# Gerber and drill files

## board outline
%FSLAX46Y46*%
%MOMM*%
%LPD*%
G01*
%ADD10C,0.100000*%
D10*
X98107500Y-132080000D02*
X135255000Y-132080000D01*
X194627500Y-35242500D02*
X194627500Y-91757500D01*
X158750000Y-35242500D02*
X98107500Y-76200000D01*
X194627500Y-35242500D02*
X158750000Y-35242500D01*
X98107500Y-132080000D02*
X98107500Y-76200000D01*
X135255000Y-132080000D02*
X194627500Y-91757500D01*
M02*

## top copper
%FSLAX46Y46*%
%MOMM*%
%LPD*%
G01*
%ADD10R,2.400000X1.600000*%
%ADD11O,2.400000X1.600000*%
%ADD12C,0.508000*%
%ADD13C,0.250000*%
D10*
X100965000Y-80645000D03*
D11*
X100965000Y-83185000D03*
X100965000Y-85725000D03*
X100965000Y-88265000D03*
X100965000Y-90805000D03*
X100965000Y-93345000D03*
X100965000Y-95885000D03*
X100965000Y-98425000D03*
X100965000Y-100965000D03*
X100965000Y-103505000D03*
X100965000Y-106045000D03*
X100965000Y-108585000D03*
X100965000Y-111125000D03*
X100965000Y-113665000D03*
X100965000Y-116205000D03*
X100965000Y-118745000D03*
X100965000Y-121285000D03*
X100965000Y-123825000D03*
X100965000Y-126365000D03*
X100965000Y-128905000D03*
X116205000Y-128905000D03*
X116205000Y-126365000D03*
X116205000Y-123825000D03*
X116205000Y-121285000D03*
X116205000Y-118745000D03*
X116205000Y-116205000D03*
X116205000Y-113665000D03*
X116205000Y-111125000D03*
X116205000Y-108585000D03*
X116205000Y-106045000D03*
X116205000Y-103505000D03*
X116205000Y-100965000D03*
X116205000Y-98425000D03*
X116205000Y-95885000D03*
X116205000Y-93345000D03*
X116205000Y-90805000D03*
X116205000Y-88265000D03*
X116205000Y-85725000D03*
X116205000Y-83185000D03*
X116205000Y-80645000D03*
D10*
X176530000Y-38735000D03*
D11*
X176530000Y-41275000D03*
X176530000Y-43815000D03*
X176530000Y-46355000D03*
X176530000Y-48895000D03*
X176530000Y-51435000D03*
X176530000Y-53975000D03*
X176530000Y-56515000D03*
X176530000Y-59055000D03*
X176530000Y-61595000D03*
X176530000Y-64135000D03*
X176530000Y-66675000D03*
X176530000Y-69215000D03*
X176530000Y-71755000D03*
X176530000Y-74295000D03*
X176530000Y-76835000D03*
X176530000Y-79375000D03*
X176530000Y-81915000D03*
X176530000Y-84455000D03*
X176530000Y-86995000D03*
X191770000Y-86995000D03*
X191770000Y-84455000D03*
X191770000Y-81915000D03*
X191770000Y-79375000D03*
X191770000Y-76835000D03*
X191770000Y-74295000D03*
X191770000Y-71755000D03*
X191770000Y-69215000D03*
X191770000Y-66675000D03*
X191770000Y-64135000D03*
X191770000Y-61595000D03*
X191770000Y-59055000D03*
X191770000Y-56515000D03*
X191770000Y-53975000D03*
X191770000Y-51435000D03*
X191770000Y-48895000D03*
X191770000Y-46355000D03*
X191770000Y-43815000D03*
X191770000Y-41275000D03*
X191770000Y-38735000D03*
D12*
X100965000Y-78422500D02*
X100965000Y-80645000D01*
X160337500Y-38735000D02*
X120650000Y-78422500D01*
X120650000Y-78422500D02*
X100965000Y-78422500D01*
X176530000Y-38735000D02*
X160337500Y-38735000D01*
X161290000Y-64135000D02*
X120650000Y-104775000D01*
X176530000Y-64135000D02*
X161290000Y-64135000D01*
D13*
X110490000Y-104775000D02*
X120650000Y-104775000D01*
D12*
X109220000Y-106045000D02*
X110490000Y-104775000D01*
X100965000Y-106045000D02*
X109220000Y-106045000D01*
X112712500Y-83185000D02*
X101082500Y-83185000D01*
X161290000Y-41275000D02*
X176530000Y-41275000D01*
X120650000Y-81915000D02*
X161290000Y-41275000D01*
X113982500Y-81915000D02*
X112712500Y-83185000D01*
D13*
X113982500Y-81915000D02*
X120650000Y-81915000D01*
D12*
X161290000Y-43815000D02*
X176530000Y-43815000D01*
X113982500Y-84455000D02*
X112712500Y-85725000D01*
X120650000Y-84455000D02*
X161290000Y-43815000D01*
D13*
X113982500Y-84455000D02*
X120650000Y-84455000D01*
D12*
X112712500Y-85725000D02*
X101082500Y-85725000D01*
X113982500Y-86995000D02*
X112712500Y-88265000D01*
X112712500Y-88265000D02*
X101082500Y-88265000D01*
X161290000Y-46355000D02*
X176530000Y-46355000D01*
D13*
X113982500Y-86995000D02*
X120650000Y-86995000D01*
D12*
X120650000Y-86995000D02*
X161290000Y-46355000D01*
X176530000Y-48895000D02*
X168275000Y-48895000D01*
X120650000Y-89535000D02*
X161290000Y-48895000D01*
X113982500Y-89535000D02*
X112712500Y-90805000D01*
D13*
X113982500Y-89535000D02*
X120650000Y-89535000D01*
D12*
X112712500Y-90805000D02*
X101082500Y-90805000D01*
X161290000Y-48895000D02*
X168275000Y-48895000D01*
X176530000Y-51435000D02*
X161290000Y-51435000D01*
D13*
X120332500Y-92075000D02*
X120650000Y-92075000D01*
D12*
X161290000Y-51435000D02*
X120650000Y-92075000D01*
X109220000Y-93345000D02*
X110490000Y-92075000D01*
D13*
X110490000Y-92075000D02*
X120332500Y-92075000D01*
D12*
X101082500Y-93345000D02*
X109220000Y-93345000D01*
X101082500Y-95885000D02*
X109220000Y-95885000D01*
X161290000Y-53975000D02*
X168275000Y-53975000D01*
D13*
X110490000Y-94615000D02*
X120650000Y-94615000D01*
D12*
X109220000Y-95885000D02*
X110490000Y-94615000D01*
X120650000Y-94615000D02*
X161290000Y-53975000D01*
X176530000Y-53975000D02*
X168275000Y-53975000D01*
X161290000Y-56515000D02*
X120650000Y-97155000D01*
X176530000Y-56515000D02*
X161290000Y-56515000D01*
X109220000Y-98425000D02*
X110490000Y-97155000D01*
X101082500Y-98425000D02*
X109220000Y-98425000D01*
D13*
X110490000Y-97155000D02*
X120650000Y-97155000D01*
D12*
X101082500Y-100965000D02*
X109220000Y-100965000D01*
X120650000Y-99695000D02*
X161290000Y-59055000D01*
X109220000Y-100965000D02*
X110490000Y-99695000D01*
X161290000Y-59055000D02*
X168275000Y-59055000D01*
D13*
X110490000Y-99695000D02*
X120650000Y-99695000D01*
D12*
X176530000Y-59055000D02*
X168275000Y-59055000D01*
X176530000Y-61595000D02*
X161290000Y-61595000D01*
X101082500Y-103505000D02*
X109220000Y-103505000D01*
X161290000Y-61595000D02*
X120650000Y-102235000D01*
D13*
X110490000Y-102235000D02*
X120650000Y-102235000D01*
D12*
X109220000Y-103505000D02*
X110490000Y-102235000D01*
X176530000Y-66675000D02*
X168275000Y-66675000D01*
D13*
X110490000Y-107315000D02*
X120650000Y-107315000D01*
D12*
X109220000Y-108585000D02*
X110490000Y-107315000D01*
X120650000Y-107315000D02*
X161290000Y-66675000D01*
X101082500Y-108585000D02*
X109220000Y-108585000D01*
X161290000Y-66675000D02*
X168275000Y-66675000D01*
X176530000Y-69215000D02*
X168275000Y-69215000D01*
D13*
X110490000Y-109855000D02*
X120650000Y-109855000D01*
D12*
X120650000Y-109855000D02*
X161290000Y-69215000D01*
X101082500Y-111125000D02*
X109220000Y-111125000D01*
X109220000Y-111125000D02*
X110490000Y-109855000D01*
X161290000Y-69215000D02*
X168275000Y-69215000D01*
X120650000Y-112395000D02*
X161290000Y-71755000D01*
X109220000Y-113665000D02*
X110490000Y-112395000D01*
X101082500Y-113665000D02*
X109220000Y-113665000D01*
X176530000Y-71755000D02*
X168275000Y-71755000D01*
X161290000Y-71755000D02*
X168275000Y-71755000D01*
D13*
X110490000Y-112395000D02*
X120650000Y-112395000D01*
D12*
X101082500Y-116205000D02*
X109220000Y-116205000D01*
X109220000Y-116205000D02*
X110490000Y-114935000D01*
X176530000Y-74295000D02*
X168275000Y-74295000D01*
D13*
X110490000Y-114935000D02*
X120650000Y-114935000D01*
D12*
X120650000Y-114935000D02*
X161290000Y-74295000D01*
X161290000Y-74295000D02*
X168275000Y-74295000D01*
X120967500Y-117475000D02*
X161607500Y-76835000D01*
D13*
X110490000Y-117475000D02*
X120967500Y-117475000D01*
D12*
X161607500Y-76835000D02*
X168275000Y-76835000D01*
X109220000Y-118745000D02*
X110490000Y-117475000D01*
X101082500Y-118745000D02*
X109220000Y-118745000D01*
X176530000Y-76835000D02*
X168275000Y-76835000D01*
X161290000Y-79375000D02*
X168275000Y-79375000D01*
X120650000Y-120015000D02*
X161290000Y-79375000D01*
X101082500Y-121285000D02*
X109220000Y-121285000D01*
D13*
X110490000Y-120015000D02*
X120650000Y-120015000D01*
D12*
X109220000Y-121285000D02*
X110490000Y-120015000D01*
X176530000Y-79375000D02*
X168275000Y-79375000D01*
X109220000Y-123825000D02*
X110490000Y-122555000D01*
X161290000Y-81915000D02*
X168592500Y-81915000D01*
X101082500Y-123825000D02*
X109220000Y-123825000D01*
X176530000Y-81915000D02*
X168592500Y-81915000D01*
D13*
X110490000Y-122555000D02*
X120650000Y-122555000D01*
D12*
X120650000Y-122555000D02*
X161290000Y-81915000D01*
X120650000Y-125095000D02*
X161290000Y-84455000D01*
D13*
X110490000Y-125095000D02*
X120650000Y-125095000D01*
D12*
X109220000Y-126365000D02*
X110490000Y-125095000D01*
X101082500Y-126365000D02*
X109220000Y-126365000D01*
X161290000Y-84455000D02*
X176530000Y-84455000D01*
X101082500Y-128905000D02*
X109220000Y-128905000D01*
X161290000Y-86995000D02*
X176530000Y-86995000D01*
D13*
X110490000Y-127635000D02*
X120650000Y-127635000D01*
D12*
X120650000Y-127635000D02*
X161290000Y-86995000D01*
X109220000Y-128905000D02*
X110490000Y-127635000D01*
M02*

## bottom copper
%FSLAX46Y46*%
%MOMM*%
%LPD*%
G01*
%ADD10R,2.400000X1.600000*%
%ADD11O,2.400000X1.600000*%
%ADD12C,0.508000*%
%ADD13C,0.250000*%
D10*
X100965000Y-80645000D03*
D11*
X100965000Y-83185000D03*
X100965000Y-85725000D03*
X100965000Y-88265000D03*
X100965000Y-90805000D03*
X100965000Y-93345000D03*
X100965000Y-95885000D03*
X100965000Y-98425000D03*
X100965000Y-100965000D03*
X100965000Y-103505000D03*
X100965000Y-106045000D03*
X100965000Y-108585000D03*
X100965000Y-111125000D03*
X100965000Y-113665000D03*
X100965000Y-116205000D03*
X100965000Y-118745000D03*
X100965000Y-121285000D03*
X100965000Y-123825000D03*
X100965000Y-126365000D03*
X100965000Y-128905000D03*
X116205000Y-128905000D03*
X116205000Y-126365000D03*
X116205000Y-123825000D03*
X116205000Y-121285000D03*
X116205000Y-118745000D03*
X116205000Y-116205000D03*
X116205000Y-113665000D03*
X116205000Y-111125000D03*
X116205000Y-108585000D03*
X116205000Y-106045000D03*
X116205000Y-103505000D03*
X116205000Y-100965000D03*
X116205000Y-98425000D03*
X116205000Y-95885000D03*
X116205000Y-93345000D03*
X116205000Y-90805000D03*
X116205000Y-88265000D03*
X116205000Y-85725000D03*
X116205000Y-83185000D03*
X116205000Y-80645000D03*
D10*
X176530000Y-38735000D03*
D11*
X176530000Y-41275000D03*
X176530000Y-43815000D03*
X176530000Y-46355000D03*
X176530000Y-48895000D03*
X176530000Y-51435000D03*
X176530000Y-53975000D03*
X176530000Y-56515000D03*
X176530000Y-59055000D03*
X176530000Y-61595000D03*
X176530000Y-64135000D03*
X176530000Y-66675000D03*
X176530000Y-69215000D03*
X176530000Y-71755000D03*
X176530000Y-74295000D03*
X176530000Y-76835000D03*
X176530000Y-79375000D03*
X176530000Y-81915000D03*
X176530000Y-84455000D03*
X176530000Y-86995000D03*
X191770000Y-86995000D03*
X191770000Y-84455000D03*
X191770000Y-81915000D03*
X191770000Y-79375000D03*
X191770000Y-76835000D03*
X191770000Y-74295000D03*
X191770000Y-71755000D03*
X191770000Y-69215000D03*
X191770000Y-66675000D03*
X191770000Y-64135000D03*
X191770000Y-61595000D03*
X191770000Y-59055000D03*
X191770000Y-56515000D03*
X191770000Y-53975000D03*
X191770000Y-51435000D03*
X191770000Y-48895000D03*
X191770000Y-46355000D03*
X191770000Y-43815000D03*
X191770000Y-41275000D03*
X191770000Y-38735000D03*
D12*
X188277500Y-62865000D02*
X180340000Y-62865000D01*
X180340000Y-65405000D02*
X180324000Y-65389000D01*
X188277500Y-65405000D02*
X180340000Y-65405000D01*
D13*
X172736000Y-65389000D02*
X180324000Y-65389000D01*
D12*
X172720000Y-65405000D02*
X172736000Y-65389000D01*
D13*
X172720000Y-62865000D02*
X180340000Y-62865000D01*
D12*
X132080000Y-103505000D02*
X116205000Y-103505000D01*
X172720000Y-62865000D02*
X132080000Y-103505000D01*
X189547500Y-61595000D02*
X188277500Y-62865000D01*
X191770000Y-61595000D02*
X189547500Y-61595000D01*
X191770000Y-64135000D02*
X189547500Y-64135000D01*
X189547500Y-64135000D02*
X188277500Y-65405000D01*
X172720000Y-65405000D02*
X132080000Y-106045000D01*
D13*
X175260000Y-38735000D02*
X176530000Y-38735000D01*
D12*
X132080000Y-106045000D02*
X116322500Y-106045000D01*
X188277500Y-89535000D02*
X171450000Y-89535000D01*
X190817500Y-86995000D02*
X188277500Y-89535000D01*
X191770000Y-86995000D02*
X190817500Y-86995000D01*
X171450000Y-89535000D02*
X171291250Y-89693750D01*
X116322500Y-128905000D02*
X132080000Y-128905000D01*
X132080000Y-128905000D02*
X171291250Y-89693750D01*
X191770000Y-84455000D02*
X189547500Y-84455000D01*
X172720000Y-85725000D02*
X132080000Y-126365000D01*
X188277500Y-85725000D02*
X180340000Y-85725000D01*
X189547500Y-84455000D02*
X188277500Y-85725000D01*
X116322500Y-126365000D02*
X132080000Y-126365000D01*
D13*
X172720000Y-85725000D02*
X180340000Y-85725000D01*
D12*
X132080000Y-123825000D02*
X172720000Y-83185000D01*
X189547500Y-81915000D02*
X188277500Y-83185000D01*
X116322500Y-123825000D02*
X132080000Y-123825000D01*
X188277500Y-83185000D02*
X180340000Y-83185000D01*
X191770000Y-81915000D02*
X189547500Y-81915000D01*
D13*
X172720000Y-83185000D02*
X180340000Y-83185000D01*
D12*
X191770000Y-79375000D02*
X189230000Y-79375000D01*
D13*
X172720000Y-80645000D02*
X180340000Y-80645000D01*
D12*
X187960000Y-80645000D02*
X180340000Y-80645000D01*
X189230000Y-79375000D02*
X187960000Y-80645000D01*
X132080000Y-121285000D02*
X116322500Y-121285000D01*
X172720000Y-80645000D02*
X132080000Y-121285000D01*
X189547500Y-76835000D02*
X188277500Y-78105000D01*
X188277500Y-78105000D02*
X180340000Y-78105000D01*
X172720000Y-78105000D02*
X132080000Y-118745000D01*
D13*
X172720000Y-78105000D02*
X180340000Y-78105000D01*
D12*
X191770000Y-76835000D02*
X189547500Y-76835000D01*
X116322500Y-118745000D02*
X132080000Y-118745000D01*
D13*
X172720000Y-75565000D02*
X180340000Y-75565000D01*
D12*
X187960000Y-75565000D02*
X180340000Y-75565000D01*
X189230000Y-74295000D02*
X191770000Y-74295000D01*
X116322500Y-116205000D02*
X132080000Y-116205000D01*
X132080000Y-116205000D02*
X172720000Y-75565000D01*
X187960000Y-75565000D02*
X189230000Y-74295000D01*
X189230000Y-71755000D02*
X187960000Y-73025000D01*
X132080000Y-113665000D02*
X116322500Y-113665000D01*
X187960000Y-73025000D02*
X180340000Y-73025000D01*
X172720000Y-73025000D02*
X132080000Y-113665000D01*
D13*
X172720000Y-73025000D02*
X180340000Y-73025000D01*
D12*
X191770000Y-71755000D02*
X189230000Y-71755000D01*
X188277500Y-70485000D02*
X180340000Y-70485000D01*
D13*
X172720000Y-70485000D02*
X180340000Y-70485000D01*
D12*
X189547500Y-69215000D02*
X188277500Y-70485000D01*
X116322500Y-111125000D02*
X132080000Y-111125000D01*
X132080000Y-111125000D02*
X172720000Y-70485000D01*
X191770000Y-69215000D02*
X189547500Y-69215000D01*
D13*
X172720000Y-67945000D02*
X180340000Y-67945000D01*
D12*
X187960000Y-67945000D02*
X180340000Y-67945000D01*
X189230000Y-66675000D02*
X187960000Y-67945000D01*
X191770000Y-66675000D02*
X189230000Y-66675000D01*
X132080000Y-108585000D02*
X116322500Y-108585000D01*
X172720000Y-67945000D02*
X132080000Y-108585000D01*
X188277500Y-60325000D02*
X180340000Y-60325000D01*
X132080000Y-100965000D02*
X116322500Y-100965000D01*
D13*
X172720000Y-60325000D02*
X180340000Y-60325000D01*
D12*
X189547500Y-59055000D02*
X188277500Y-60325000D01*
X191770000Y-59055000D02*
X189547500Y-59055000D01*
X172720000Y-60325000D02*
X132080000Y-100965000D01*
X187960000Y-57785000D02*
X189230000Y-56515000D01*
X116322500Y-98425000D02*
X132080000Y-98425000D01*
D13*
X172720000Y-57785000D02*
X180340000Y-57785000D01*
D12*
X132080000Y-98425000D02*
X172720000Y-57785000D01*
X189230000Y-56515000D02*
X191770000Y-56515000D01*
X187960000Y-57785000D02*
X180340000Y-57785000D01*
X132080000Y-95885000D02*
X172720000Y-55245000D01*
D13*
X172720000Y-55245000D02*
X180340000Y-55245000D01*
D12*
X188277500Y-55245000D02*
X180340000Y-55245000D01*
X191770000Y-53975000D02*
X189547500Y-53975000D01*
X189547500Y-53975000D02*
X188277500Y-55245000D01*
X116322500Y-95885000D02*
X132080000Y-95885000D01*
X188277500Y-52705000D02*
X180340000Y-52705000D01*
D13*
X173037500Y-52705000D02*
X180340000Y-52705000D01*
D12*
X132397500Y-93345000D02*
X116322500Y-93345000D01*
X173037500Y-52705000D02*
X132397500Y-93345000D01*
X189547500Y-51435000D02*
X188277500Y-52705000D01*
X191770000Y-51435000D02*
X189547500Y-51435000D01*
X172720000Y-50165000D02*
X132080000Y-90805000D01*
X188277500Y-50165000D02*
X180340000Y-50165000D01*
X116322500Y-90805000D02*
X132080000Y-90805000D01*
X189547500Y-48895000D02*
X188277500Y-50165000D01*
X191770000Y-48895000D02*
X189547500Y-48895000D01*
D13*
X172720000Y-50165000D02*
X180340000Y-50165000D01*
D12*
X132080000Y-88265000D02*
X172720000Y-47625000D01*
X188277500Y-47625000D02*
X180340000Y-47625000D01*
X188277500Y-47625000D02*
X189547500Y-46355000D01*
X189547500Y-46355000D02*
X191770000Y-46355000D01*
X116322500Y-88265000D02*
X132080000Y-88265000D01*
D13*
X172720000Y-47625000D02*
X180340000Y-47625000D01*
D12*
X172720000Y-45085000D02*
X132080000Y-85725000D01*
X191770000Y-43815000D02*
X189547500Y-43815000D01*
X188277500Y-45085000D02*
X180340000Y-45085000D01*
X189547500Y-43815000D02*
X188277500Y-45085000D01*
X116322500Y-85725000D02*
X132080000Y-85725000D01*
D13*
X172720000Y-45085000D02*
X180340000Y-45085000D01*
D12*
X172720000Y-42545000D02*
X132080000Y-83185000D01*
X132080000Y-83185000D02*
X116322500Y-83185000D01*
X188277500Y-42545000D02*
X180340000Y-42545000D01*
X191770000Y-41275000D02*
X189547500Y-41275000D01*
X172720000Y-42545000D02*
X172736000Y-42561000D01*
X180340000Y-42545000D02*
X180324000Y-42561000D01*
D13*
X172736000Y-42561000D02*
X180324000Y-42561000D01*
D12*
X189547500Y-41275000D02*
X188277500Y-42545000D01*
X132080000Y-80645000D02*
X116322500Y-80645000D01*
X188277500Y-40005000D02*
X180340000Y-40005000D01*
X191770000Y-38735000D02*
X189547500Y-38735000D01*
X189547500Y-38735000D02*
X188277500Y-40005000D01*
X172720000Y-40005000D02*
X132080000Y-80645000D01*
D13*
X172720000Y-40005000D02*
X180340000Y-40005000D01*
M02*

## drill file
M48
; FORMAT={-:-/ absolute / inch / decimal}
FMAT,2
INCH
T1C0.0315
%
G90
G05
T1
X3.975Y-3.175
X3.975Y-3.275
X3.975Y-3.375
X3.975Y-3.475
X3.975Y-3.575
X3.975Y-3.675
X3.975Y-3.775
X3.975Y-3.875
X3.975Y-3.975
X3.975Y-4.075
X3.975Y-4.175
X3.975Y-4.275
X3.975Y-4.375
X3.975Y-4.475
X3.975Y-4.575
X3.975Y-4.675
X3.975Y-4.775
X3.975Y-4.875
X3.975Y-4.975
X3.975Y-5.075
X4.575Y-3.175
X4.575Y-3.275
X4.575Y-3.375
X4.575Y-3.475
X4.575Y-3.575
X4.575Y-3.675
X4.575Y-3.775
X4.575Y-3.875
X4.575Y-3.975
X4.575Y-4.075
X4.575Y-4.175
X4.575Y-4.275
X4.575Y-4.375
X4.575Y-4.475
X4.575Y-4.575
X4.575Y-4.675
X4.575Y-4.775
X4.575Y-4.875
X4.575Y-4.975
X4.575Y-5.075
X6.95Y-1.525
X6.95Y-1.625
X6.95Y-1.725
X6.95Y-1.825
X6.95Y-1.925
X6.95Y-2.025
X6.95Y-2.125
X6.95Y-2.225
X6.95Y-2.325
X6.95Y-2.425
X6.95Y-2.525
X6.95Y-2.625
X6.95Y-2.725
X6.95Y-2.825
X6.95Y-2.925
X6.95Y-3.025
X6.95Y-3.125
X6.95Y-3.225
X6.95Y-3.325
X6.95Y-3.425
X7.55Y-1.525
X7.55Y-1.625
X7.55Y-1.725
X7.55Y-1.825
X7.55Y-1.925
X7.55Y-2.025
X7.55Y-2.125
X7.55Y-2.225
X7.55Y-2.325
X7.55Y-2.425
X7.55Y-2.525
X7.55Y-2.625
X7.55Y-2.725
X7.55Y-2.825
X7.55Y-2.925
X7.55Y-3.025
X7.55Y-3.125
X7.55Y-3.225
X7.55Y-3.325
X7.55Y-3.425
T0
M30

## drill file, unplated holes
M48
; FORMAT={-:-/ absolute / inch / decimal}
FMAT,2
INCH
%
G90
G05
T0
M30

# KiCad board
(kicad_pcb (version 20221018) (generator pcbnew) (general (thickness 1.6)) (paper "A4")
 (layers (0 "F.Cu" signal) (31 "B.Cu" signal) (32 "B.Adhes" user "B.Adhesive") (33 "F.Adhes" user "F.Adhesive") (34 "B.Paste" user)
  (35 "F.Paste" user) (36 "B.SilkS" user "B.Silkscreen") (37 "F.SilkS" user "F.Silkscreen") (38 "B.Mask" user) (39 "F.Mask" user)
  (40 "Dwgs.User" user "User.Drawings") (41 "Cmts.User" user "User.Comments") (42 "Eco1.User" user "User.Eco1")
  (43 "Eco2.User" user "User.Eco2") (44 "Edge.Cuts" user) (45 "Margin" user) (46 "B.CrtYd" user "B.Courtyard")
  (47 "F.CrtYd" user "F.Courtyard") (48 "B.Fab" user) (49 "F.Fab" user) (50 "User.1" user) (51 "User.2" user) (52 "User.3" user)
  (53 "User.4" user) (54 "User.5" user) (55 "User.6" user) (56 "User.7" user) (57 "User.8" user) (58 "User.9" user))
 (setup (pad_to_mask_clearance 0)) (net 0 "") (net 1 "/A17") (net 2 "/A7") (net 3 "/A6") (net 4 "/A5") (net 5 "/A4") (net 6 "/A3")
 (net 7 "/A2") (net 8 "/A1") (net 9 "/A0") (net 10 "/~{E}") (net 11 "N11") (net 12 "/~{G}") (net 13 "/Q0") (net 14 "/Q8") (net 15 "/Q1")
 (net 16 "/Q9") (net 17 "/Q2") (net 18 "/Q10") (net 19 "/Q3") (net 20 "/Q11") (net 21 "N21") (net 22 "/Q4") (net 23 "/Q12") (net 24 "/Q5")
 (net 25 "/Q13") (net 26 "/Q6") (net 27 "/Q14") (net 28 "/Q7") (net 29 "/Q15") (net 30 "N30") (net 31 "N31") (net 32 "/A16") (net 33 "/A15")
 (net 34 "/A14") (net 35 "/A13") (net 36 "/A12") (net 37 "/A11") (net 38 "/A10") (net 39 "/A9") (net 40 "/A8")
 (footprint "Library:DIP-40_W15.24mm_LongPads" (layer "F.Cu") (at 176.53 38.735)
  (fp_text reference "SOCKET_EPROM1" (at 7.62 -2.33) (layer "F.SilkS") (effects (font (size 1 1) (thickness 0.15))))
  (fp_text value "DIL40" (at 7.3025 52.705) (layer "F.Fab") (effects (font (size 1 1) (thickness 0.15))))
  (pad "1" thru_hole rect (at 0 0) (size 2.4 1.6) (drill 0.8) (layers "*.Cu" "*.Mask") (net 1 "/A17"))
  (pad "2" thru_hole oval (at 0 2.54) (size 2.4 1.6) (drill 0.8) (layers "*.Cu" "*.Mask") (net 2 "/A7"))
  (pad "3" thru_hole oval (at 0 5.08) (size 2.4 1.6) (drill 0.8) (layers "*.Cu" "*.Mask") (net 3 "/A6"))
  (pad "4" thru_hole oval (at 0 7.62) (size 2.4 1.6) (drill 0.8) (layers "*.Cu" "*.Mask") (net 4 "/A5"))
  (pad "5" thru_hole oval (at 0 10.16) (size 2.4 1.6) (drill 0.8) (layers "*.Cu" "*.Mask") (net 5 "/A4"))
  (pad "6" thru_hole oval (at 0 12.7) (size 2.4 1.6) (drill 0.8) (layers "*.Cu" "*.Mask") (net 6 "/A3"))
  (pad "7" thru_hole oval (at 0 15.24) (size 2.4 1.6) (drill 0.8) (layers "*.Cu" "*.Mask") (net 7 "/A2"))
  (pad "8" thru_hole oval (at 0 17.78) (size 2.4 1.6) (drill 0.8) (layers "*.Cu" "*.Mask") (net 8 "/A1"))
  (pad "9" thru_hole oval (at 0 20.32) (size 2.4 1.6) (drill 0.8) (layers "*.Cu" "*.Mask") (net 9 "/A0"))
  (pad "10" thru_hole oval (at 0 22.86) (size 2.4 1.6) (drill 0.8) (layers "*.Cu" "*.Mask") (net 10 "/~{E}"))
  (pad "11" thru_hole oval (at 0 25.4) (size 2.4 1.6) (drill 0.8) (layers "*.Cu" "*.Mask") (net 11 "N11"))
  (pad "12" thru_hole oval (at 0 27.94) (size 2.4 1.6) (drill 0.8) (layers "*.Cu" "*.Mask") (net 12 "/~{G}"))
  (pad "13" thru_hole oval (at 0 30.48) (size 2.4 1.6) (drill 0.8) (layers "*.Cu" "*.Mask") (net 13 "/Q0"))
  (pad "14" thru_hole oval (at 0 33.02) (size 2.4 1.6) (drill 0.8) (layers "*.Cu" "*.Mask") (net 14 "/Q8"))
  (pad "15" thru_hole oval (at 0 35.56) (size 2.4 1.6) (drill 0.8) (layers "*.Cu" "*.Mask") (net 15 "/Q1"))
  (pad "16" thru_hole oval (at 0 38.1) (size 2.4 1.6) (drill 0.8) (layers "*.Cu" "*.Mask") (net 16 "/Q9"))
  (pad "17" thru_hole oval (at 0 40.64) (size 2.4 1.6) (drill 0.8) (layers "*.Cu" "*.Mask") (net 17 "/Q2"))
  (pad "18" thru_hole oval (at 0 43.18) (size 2.4 1.6) (drill 0.8) (layers "*.Cu" "*.Mask") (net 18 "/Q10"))
  (pad "19" thru_hole oval (at 0 45.72) (size 2.4 1.6) (drill 0.8) (layers "*.Cu" "*.Mask") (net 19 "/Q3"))
  (pad "20" thru_hole oval (at 0 48.26) (size 2.4 1.6) (drill 0.8) (layers "*.Cu" "*.Mask") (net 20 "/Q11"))
  (pad "21" thru_hole oval (at 15.24 48.26) (size 2.4 1.6) (drill 0.8) (layers "*.Cu" "*.Mask") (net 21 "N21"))
  (pad "22" thru_hole oval (at 15.24 45.72) (size 2.4 1.6) (drill 0.8) (layers "*.Cu" "*.Mask") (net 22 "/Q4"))
  (pad "23" thru_hole oval (at 15.24 43.18) (size 2.4 1.6) (drill 0.8) (layers "*.Cu" "*.Mask") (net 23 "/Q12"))
  (pad "24" thru_hole oval (at 15.24 40.64) (size 2.4 1.6) (drill 0.8) (layers "*.Cu" "*.Mask") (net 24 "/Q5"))
  (pad "25" thru_hole oval (at 15.24 38.1) (size 2.4 1.6) (drill 0.8) (layers "*.Cu" "*.Mask") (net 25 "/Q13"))
  (pad "26" thru_hole oval (at 15.24 35.56) (size 2.4 1.6) (drill 0.8) (layers "*.Cu" "*.Mask") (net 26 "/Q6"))
  (pad "27" thru_hole oval (at 15.24 33.02) (size 2.4 1.6) (drill 0.8) (layers "*.Cu" "*.Mask") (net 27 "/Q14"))
  (pad "28" thru_hole oval (at 15.24 30.48) (size 2.4 1.6) (drill 0.8) (layers "*.Cu" "*.Mask") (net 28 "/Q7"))
  (pad "29" thru_hole oval (at 15.24 27.94) (size 2.4 1.6) (drill 0.8) (layers "*.Cu" "*.Mask") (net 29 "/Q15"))
  (pad "30" thru_hole oval (at 15.24 25.4) (size 2.4 1.6) (drill 0.8) (layers "*.Cu" "*.Mask") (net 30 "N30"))
  (pad "31" thru_hole oval (at 15.24 22.86) (size 2.4 1.6) (drill 0.8) (layers "*.Cu" "*.Mask") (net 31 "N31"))
  (pad "32" thru_hole oval (at 15.24 20.32) (size 2.4 1.6) (drill 0.8) (layers "*.Cu" "*.Mask") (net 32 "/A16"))
  (pad "33" thru_hole oval (at 15.24 17.78) (size 2.4 1.6) (drill 0.8) (layers "*.Cu" "*.Mask") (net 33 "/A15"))
  (pad "34" thru_hole oval (at 15.24 15.24) (size 2.4 1.6) (drill 0.8) (layers "*.Cu" "*.Mask") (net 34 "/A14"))
  (pad "35" thru_hole oval (at 15.24 12.7) (size 2.4 1.6) (drill 0.8) (layers "*.Cu" "*.Mask") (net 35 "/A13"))
  (pad "36" thru_hole oval (at 15.24 10.16) (size 2.4 1.6) (drill 0.8) (layers "*.Cu" "*.Mask") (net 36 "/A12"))
  (pad "37" thru_hole oval (at 15.24 7.62) (size 2.4 1.6) (drill 0.8) (layers "*.Cu" "*.Mask") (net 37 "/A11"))
  (pad "38" thru_hole oval (at 15.24 5.08) (size 2.4 1.6) (drill 0.8) (layers "*.Cu" "*.Mask") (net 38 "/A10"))
  (pad "39" thru_hole oval (at 15.24 2.54) (size 2.4 1.6) (drill 0.8) (layers "*.Cu" "*.Mask") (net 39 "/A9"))
  (pad "40" thru_hole oval (at 15.24 0) (size 2.4 1.6) (drill 0.8) (layers "*.Cu" "*.Mask") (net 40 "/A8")))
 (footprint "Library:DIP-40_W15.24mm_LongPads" (layer "F.Cu") (at 100.965 80.645)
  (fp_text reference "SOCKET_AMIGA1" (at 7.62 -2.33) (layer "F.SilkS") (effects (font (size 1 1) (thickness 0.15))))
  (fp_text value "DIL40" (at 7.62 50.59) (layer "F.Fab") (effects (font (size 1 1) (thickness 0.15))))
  (pad "1" thru_hole rect (at 0 0) (size 2.4 1.6) (drill 0.8) (layers "*.Cu" "*.Mask") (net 1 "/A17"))
  (pad "2" thru_hole oval (at 0 2.54) (size 2.4 1.6) (drill 0.8) (layers "*.Cu" "*.Mask") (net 2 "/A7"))
  (pad "3" thru_hole oval (at 0 5.08) (size 2.4 1.6) (drill 0.8) (layers "*.Cu" "*.Mask") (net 3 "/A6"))
  (pad "4" thru_hole oval (at 0 7.62) (size 2.4 1.6) (drill 0.8) (layers "*.Cu" "*.Mask") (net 4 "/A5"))
  (pad "5" thru_hole oval (at 0 10.16) (size 2.4 1.6) (drill 0.8) (layers "*.Cu" "*.Mask") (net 5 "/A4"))
  (pad "6" thru_hole oval (at 0 12.7) (size 2.4 1.6) (drill 0.8) (layers "*.Cu" "*.Mask") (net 6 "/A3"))
  (pad "7" thru_hole oval (at 0 15.24) (size 2.4 1.6) (drill 0.8) (layers "*.Cu" "*.Mask") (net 7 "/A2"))
  (pad "8" thru_hole oval (at 0 17.78) (size 2.4 1.6) (drill 0.8) (layers "*.Cu" "*.Mask") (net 8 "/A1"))
  (pad "9" thru_hole oval (at 0 20.32) (size 2.4 1.6) (drill 0.8) (layers "*.Cu" "*.Mask") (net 9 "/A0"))
  (pad "10" thru_hole oval (at 0 22.86) (size 2.4 1.6) (drill 0.8) (layers "*.Cu" "*.Mask") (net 10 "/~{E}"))
  (pad "11" thru_hole oval (at 0 25.4) (size 2.4 1.6) (drill 0.8) (layers "*.Cu" "*.Mask") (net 11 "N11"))
  (pad "12" thru_hole oval (at 0 27.94) (size 2.4 1.6) (drill 0.8) (layers "*.Cu" "*.Mask") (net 12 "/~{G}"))
  (pad "13" thru_hole oval (at 0 30.48) (size 2.4 1.6) (drill 0.8) (layers "*.Cu" "*.Mask") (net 13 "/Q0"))
  (pad "14" thru_hole oval (at 0 33.02) (size 2.4 1.6) (drill 0.8) (layers "*.Cu" "*.Mask") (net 14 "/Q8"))
  (pad "15" thru_hole oval (at 0 35.56) (size 2.4 1.6) (drill 0.8) (layers "*.Cu" "*.Mask") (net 15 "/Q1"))
  (pad "16" thru_hole oval (at 0 38.1) (size 2.4 1.6) (drill 0.8) (layers "*.Cu" "*.Mask") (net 16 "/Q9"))
  (pad "17" thru_hole oval (at 0 40.64) (size 2.4 1.6) (drill 0.8) (layers "*.Cu" "*.Mask") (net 17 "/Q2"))
  (pad "18" thru_hole oval (at 0 43.18) (size 2.4 1.6) (drill 0.8) (layers "*.Cu" "*.Mask") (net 18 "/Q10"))
  (pad "19" thru_hole oval (at 0 45.72) (size 2.4 1.6) (drill 0.8) (layers "*.Cu" "*.Mask") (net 19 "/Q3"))
  (pad "20" thru_hole oval (at 0 48.26) (size 2.4 1.6) (drill 0.8) (layers "*.Cu" "*.Mask") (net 20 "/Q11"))
  (pad "21" thru_hole oval (at 15.24 48.26) (size 2.4 1.6) (drill 0.8) (layers "*.Cu" "*.Mask") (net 21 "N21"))
  (pad "22" thru_hole oval (at 15.24 45.72) (size 2.4 1.6) (drill 0.8) (layers "*.Cu" "*.Mask") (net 22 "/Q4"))
  (pad "23" thru_hole oval (at 15.24 43.18) (size 2.4 1.6) (drill 0.8) (layers "*.Cu" "*.Mask") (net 23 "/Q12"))
  (pad "24" thru_hole oval (at 15.24 40.64) (size 2.4 1.6) (drill 0.8) (layers "*.Cu" "*.Mask") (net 24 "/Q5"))
  (pad "25" thru_hole oval (at 15.24 38.1) (size 2.4 1.6) (drill 0.8) (layers "*.Cu" "*.Mask") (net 25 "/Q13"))
  (pad "26" thru_hole oval (at 15.24 35.56) (size 2.4 1.6) (drill 0.8) (layers "*.Cu" "*.Mask") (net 26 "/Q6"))
  (pad "27" thru_hole oval (at 15.24 33.02) (size 2.4 1.6) (drill 0.8) (layers "*.Cu" "*.Mask") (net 27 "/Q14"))
  (pad "28" thru_hole oval (at 15.24 30.48) (size 2.4 1.6) (drill 0.8) (layers "*.Cu" "*.Mask") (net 28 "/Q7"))
  (pad "29" thru_hole oval (at 15.24 27.94) (size 2.4 1.6) (drill 0.8) (layers "*.Cu" "*.Mask") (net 29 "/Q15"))
  (pad "30" thru_hole oval (at 15.24 25.4) (size 2.4 1.6) (drill 0.8) (layers "*.Cu" "*.Mask") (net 30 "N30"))
  (pad "31" thru_hole oval (at 15.24 22.86) (size 2.4 1.6) (drill 0.8) (layers "*.Cu" "*.Mask") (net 31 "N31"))
  (pad "32" thru_hole oval (at 15.24 20.32) (size 2.4 1.6) (drill 0.8) (layers "*.Cu" "*.Mask") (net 32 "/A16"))
  (pad "33" thru_hole oval (at 15.24 17.78) (size 2.4 1.6) (drill 0.8) (layers "*.Cu" "*.Mask") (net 33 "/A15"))
  (pad "34" thru_hole oval (at 15.24 15.24) (size 2.4 1.6) (drill 0.8) (layers "*.Cu" "*.Mask") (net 34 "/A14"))
  (pad "35" thru_hole oval (at 15.24 12.7) (size 2.4 1.6) (drill 0.8) (layers "*.Cu" "*.Mask") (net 35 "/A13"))
  (pad "36" thru_hole oval (at 15.24 10.16) (size 2.4 1.6) (drill 0.8) (layers "*.Cu" "*.Mask") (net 36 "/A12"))
  (pad "37" thru_hole oval (at 15.24 7.62) (size 2.4 1.6) (drill 0.8) (layers "*.Cu" "*.Mask") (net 37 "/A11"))
  (pad "38" thru_hole oval (at 15.24 5.08) (size 2.4 1.6) (drill 0.8) (layers "*.Cu" "*.Mask") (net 38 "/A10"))
  (pad "39" thru_hole oval (at 15.24 2.54) (size 2.4 1.6) (drill 0.8) (layers "*.Cu" "*.Mask") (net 39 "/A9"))
  (pad "40" thru_hole oval (at 15.24 0) (size 2.4 1.6) (drill 0.8) (layers "*.Cu" "*.Mask") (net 40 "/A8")))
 (gr_line (start 98.1075 132.08) (end 135.255 132.08) (stroke (width 0.1) (type solid)) (layer "Edge.Cuts"))
 (gr_line (start 194.6275 35.2425) (end 194.6275 91.7575) (stroke (width 0.1) (type default)) (layer "Edge.Cuts"))
 (gr_line (start 158.75 35.2425) (end 98.1075 76.2) (stroke (width 0.1) (type default)) (layer "Edge.Cuts"))
 (gr_line (start 194.6275 35.2425) (end 158.75 35.2425) (stroke (width 0.1) (type default)) (layer "Edge.Cuts"))
 (gr_line (start 98.1075 132.08) (end 98.1075 76.2) (stroke (width 0.1) (type default)) (layer "Edge.Cuts"))
 (gr_line (start 135.255 132.08) (end 194.6275 91.7575) (stroke (width 0.1) (type default)) (layer "Edge.Cuts"))
 (segment (start 176.53 38.735) (end 160.3375 38.735) (width 0.508) (layer "F.Cu") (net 1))
 (segment (start 120.65 78.4225) (end 100.965 78.4225) (width 0.508) (layer "F.Cu") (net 1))
 (segment (start 100.965 78.4225) (end 100.965 80.645) (width 0.508) (layer "F.Cu") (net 1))
 (segment (start 160.3375 38.735) (end 120.65 78.4225) (width 0.508) (layer "F.Cu") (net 1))
 (segment (start 175.26 38.735) (end 176.53 38.735) (width 0.25) (layer "B.Cu") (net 1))
 (segment (start 112.7125 83.185) (end 101.0825 83.185) (width 0.508) (layer "F.Cu") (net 2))
 (segment (start 161.29 41.275) (end 176.53 41.275) (width 0.508) (layer "F.Cu") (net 2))
 (segment (start 120.65 81.915) (end 161.29 41.275) (width 0.508) (layer "F.Cu") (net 2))
 (segment (start 113.9825 81.915) (end 112.7125 83.185) (width 0.508) (layer "F.Cu") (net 2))
 (segment (start 113.9825 81.915) (end 120.65 81.915) (width 0.25) (layer "F.Cu") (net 2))
 (segment (start 161.29 43.815) (end 176.53 43.815) (width 0.508) (layer "F.Cu") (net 3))
 (segment (start 113.9825 84.455) (end 112.7125 85.725) (width 0.508) (layer "F.Cu") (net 3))
 (segment (start 120.65 84.455) (end 161.29 43.815) (width 0.508) (layer "F.Cu") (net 3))
 (segment (start 113.9825 84.455) (end 120.65 84.455) (width 0.25) (layer "F.Cu") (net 3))
 (segment (start 112.7125 85.725) (end 101.0825 85.725) (width 0.508) (layer "F.Cu") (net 3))
 (segment (start 113.9825 86.995) (end 112.7125 88.265) (width 0.508) (layer "F.Cu") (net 4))
 (segment (start 112.7125 88.265) (end 101.0825 88.265) (width 0.508) (layer "F.Cu") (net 4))
 (segment (start 161.29 46.355) (end 176.53 46.355) (width 0.508) (layer "F.Cu") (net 4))
 (segment (start 113.9825 86.995) (end 120.65 86.995) (width 0.25) (layer "F.Cu") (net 4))
 (segment (start 120.65 86.995) (end 161.29 46.355) (width 0.508) (layer "F.Cu") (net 4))
 (segment (start 176.53 48.895) (end 168.275 48.895) (width 0.508) (layer "F.Cu") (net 5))
 (segment (start 120.65 89.535) (end 161.29 48.895) (width 0.508) (layer "F.Cu") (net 5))
 (segment (start 113.9825 89.535) (end 112.7125 90.805) (width 0.508) (layer "F.Cu") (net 5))
 (segment (start 113.9825 89.535) (end 120.65 89.535) (width 0.25) (layer "F.Cu") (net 5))
 (segment (start 112.7125 90.805) (end 101.0825 90.805) (width 0.508) (layer "F.Cu") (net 5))
 (segment (start 161.29 48.895) (end 168.275 48.895) (width 0.508) (layer "F.Cu") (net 5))
 (segment (start 176.53 51.435) (end 161.29 51.435) (width 0.508) (layer "F.Cu") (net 6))
 (segment (start 120.3325 92.075) (end 120.65 92.075) (width 0.25) (layer "F.Cu") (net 6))
 (segment (start 161.29 51.435) (end 120.65 92.075) (width 0.508) (layer "F.Cu") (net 6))
 (segment (start 109.22 93.345) (end 110.49 92.075) (width 0.508) (layer "F.Cu") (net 6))
 (segment (start 110.49 92.075) (end 120.3325 92.075) (width 0.25) (layer "F.Cu") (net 6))
 (segment (start 101.0825 93.345) (end 109.22 93.345) (width 0.508) (layer "F.Cu") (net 6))
 (segment (start 101.0825 95.885) (end 109.22 95.885) (width 0.508) (layer "F.Cu") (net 7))
 (segment (start 161.29 53.975) (end 168.275 53.975) (width 0.508) (layer "F.Cu") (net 7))
 (segment (start 110.49 94.615) (end 120.65 94.615) (width 0.25) (layer "F.Cu") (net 7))
 (segment (start 109.22 95.885) (end 110.49 94.615) (width 0.508) (layer "F.Cu") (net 7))
 (segment (start 120.65 94.615) (end 161.29 53.975) (width 0.508) (layer "F.Cu") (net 7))
 (segment (start 176.53 53.975) (end 168.275 53.975) (width 0.508) (layer "F.Cu") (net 7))
 (segment (start 161.29 56.515) (end 120.65 97.155) (width 0.508) (layer "F.Cu") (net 8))
 (segment (start 176.53 56.515) (end 161.29 56.515) (width 0.508) (layer "F.Cu") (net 8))
 (segment (start 109.22 98.425) (end 110.49 97.155) (width 0.508) (layer "F.Cu") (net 8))
 (segment (start 101.0825 98.425) (end 109.22 98.425) (width 0.508) (layer "F.Cu") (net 8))
 (segment (start 110.49 97.155) (end 120.65 97.155) (width 0.25) (layer "F.Cu") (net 8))
 (segment (start 101.0825 100.965) (end 109.22 100.965) (width 0.508) (layer "F.Cu") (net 9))
 (segment (start 120.65 99.695) (end 161.29 59.055) (width 0.508) (layer "F.Cu") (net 9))
 (segment (start 109.22 100.965) (end 110.49 99.695) (width 0.508) (layer "F.Cu") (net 9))
 (segment (start 161.29 59.055) (end 168.275 59.055) (width 0.508) (layer "F.Cu") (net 9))
 (segment (start 110.49 99.695) (end 120.65 99.695) (width 0.25) (layer "F.Cu") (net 9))
 (segment (start 176.53 59.055) (end 168.275 59.055) (width 0.508) (layer "F.Cu") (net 9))
 (segment (start 176.53 61.595) (end 161.29 61.595) (width 0.508) (layer "F.Cu") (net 10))
 (segment (start 101.0825 103.505) (end 109.22 103.505) (width 0.508) (layer "F.Cu") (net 10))
 (segment (start 161.29 61.595) (end 120.65 102.235) (width 0.508) (layer "F.Cu") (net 10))
 (segment (start 110.49 102.235) (end 120.65 102.235) (width 0.25) (layer "F.Cu") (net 10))
 (segment (start 109.22 103.505) (end 110.49 102.235) (width 0.508) (layer "F.Cu") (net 10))
 (segment (start 100.965 106.045) (end 109.22 106.045) (width 0.508) (layer "F.Cu") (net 11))
 (segment (start 176.53 64.135) (end 161.29 64.135) (width 0.508) (layer "F.Cu") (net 11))
 (segment (start 110.49 104.775) (end 120.65 104.775) (width 0.25) (layer "F.Cu") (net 11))
 (segment (start 109.22 106.045) (end 110.49 104.775) (width 0.508) (layer "F.Cu") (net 11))
 (segment (start 161.29 64.135) (end 120.65 104.775) (width 0.508) (layer "F.Cu") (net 11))
 (segment (start 176.53 66.675) (end 168.275 66.675) (width 0.508) (layer "F.Cu") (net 12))
 (segment (start 110.49 107.315) (end 120.65 107.315) (width 0.25) (layer "F.Cu") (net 12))
 (segment (start 109.22 108.585) (end 110.49 107.315) (width 0.508) (layer "F.Cu") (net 12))
 (segment (start 120.65 107.315) (end 161.29 66.675) (width 0.508) (layer "F.Cu") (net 12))
 (segment (start 101.0825 108.585) (end 109.22 108.585) (width 0.508) (layer "F.Cu") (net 12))
 (segment (start 161.29 66.675) (end 168.275 66.675) (width 0.508) (layer "F.Cu") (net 12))
 (segment (start 176.53 69.215) (end 168.275 69.215) (width 0.508) (layer "F.Cu") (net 13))
 (segment (start 110.49 109.855) (end 120.65 109.855) (width 0.25) (layer "F.Cu") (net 13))
 (segment (start 120.65 109.855) (end 161.29 69.215) (width 0.508) (layer "F.Cu") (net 13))
 (segment (start 101.0825 111.125) (end 109.22 111.125) (width 0.508) (layer "F.Cu") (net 13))
 (segment (start 109.22 111.125) (end 110.49 109.855) (width 0.508) (layer "F.Cu") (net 13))
 (segment (start 161.29 69.215) (end 168.275 69.215) (width 0.508) (layer "F.Cu") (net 13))
 (segment (start 120.65 112.395) (end 161.29 71.755) (width 0.508) (layer "F.Cu") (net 14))
 (segment (start 109.22 113.665) (end 110.49 112.395) (width 0.508) (layer "F.Cu") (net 14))
 (segment (start 101.0825 113.665) (end 109.22 113.665) (width 0.508) (layer "F.Cu") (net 14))
 (segment (start 176.53 71.755) (end 168.275 71.755) (width 0.508) (layer "F.Cu") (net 14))
 (segment (start 161.29 71.755) (end 168.275 71.755) (width 0.508) (layer "F.Cu") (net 14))
 (segment (start 110.49 112.395) (end 120.65 112.395) (width 0.25) (layer "F.Cu") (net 14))
 (segment (start 101.0825 116.205) (end 109.22 116.205) (width 0.508) (layer "F.Cu") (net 15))
 (segment (start 109.22 116.205) (end 110.49 114.935) (width 0.508) (layer "F.Cu") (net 15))
 (segment (start 176.53 74.295) (end 168.275 74.295) (width 0.508) (layer "F.Cu") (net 15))
 (segment (start 110.49 114.935) (end 120.65 114.935) (width 0.25) (layer "F.Cu") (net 15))
 (segment (start 120.65 114.935) (end 161.29 74.295) (width 0.508) (layer "F.Cu") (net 15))
 (segment (start 161.29 74.295) (end 168.275 74.295) (width 0.508) (layer "F.Cu") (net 15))
 (segment (start 120.9675 117.475) (end 161.6075 76.835) (width 0.508) (layer "F.Cu") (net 16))
 (segment (start 110.49 117.475) (end 120.9675 117.475) (width 0.25) (layer "F.Cu") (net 16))
 (segment (start 161.6075 76.835) (end 168.275 76.835) (width 0.508) (layer "F.Cu") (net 16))
 (segment (start 109.22 118.745) (end 110.49 117.475) (width 0.508) (layer "F.Cu") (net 16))
 (segment (start 101.0825 118.745) (end 109.22 118.745) (width 0.508) (layer "F.Cu") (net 16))
 (segment (start 176.53 76.835) (end 168.275 76.835) (width 0.508) (layer "F.Cu") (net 16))
 (segment (start 161.29 79.375) (end 168.275 79.375) (width 0.508) (layer "F.Cu") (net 17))
 (segment (start 120.65 120.015) (end 161.29 79.375) (width 0.508) (layer "F.Cu") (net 17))
 (segment (start 101.0825 121.285) (end 109.22 121.285) (width 0.508) (layer "F.Cu") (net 17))
 (segment (start 110.49 120.015) (end 120.65 120.015) (width 0.25) (layer "F.Cu") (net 17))
 (segment (start 109.22 121.285) (end 110.49 120.015) (width 0.508) (layer "F.Cu") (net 17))
 (segment (start 176.53 79.375) (end 168.275 79.375) (width 0.508) (layer "F.Cu") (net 17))
 (segment (start 109.22 123.825) (end 110.49 122.555) (width 0.508) (layer "F.Cu") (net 18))
 (segment (start 161.29 81.915) (end 168.5925 81.915) (width 0.508) (layer "F.Cu") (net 18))
 (segment (start 101.0825 123.825) (end 109.22 123.825) (width 0.508) (layer "F.Cu") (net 18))
 (segment (start 176.53 81.915) (end 168.5925 81.915) (width 0.508) (layer "F.Cu") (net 18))
 (segment (start 110.49 122.555) (end 120.65 122.555) (width 0.25) (layer "F.Cu") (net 18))
 (segment (start 120.65 122.555) (end 161.29 81.915) (width 0.508) (layer "F.Cu") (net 18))
 (segment (start 120.65 125.095) (end 161.29 84.455) (width 0.508) (layer "F.Cu") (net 19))
 (segment (start 110.49 125.095) (end 120.65 125.095) (width 0.25) (layer "F.Cu") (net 19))
 (segment (start 109.22 126.365) (end 110.49 125.095) (width 0.508) (layer "F.Cu") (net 19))
 (segment (start 101.0825 126.365) (end 109.22 126.365) (width 0.508) (layer "F.Cu") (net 19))
 (segment (start 161.29 84.455) (end 176.53 84.455) (width 0.508) (layer "F.Cu") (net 19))
 (segment (start 101.0825 128.905) (end 109.22 128.905) (width 0.508) (layer "F.Cu") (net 20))
 (segment (start 161.29 86.995) (end 176.53 86.995) (width 0.508) (layer "F.Cu") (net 20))
 (segment (start 110.49 127.635) (end 120.65 127.635) (width 0.25) (layer "F.Cu") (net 20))
 (segment (start 120.65 127.635) (end 161.29 86.995) (width 0.508) (layer "F.Cu") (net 20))
 (segment (start 109.22 128.905) (end 110.49 127.635) (width 0.508) (layer "F.Cu") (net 20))
 (segment (start 188.2775 89.535) (end 171.45 89.535) (width 0.508) (layer "B.Cu") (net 21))
 (segment (start 190.8175 86.995) (end 188.2775 89.535) (width 0.508) (layer "B.Cu") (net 21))
 (segment (start 191.77 86.995) (end 190.8175 86.995) (width 0.508) (layer "B.Cu") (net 21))
 (segment (start 171.45 89.535) (end 171.29125 89.69375) (width 0.508) (layer "B.Cu") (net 21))
 (segment (start 116.3225 128.905) (end 132.08 128.905) (width 0.508) (layer "B.Cu") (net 21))
 (segment (start 132.08 128.905) (end 171.29125 89.69375) (width 0.508) (layer "B.Cu") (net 21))
 (segment (start 191.77 84.455) (end 189.5475 84.455) (width 0.508) (layer "B.Cu") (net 22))
 (segment (start 172.72 85.725) (end 132.08 126.365) (width 0.508) (layer "B.Cu") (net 22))
 (segment (start 188.2775 85.725) (end 180.34 85.725) (width 0.508) (layer "B.Cu") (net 22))
 (segment (start 189.5475 84.455) (end 188.2775 85.725) (width 0.508) (layer "B.Cu") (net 22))
 (segment (start 116.3225 126.365) (end 132.08 126.365) (width 0.508) (layer "B.Cu") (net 22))
 (segment (start 172.72 85.725) (end 180.34 85.725) (width 0.25) (layer "B.Cu") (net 22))
 (segment (start 132.08 123.825) (end 172.72 83.185) (width 0.508) (layer "B.Cu") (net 23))
 (segment (start 189.5475 81.915) (end 188.2775 83.185) (width 0.508) (layer "B.Cu") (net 23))
 (segment (start 116.3225 123.825) (end 132.08 123.825) (width 0.508) (layer "B.Cu") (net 23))
 (segment (start 188.2775 83.185) (end 180.34 83.185) (width 0.508) (layer "B.Cu") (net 23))
 (segment (start 191.77 81.915) (end 189.5475 81.915) (width 0.508) (layer "B.Cu") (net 23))
 (segment (start 172.72 83.185) (end 180.34 83.185) (width 0.25) (layer "B.Cu") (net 23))
 (segment (start 191.77 79.375) (end 189.23 79.375) (width 0.508) (layer "B.Cu") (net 24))
 (segment (start 172.72 80.645) (end 180.34 80.645) (width 0.25) (layer "B.Cu") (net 24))
 (segment (start 187.96 80.645) (end 180.34 80.645) (width 0.508) (layer "B.Cu") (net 24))
 (segment (start 189.23 79.375) (end 187.96 80.645) (width 0.508) (layer "B.Cu") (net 24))
 (segment (start 132.08 121.285) (end 116.3225 121.285) (width 0.508) (layer "B.Cu") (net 24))
 (segment (start 172.72 80.645) (end 132.08 121.285) (width 0.508) (layer "B.Cu") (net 24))
 (segment (start 189.5475 76.835) (end 188.2775 78.105) (width 0.508) (layer "B.Cu") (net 25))
 (segment (start 188.2775 78.105) (end 180.34 78.105) (width 0.508) (layer "B.Cu") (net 25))
 (segment (start 172.72 78.105) (end 132.08 118.745) (width 0.508) (layer "B.Cu") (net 25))
 (segment (start 172.72 78.105) (end 180.34 78.105) (width 0.25) (layer "B.Cu") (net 25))
 (segment (start 191.77 76.835) (end 189.5475 76.835) (width 0.508) (layer "B.Cu") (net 25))
 (segment (start 116.3225 118.745) (end 132.08 118.745) (width 0.508) (layer "B.Cu") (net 25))
 (segment (start 172.72 75.565) (end 180.34 75.565) (width 0.25) (layer "B.Cu") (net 26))
 (segment (start 187.96 75.565) (end 180.34 75.565) (width 0.508) (layer "B.Cu") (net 26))
 (segment (start 189.23 74.295) (end 191.77 74.295) (width 0.508) (layer "B.Cu") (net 26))
 (segment (start 116.3225 116.205) (end 132.08 116.205) (width 0.508) (layer "B.Cu") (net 26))
 (segment (start 132.08 116.205) (end 172.72 75.565) (width 0.508) (layer "B.Cu") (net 26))
 (segment (start 187.96 75.565) (end 189.23 74.295) (width 0.508) (layer "B.Cu") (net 26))
 (segment (start 189.23 71.755) (end 187.96 73.025) (width 0.508) (layer "B.Cu") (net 27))
 (segment (start 132.08 113.665) (end 116.3225 113.665) (width 0.508) (layer "B.Cu") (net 27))
 (segment (start 187.96 73.025) (end 180.34 73.025) (width 0.508) (layer "B.Cu") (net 27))
 (segment (start 172.72 73.025) (end 132.08 113.665) (width 0.508) (layer "B.Cu") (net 27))
 (segment (start 172.72 73.025) (end 180.34 73.025) (width 0.25) (layer "B.Cu") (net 27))
 (segment (start 191.77 71.755) (end 189.23 71.755) (width 0.508) (layer "B.Cu") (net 27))
 (segment (start 188.2775 70.485) (end 180.34 70.485) (width 0.508) (layer "B.Cu") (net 28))
 (segment (start 172.72 70.485) (end 180.34 70.485) (width 0.25) (layer "B.Cu") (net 28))
 (segment (start 189.5475 69.215) (end 188.2775 70.485) (width 0.508) (layer "B.Cu") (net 28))
 (segment (start 116.3225 111.125) (end 132.08 111.125) (width 0.508) (layer "B.Cu") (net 28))
 (segment (start 132.08 111.125) (end 172.72 70.485) (width 0.508) (layer "B.Cu") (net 28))
 (segment (start 191.77 69.215) (end 189.5475 69.215) (width 0.508) (layer "B.Cu") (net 28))
 (segment (start 172.72 67.945) (end 180.34 67.945) (width 0.25) (layer "B.Cu") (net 29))
 (segment (start 187.96 67.945) (end 180.34 67.945) (width 0.508) (layer "B.Cu") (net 29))
 (segment (start 189.23 66.675) (end 187.96 67.945) (width 0.508) (layer "B.Cu") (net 29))
 (segment (start 191.77 66.675) (end 189.23 66.675) (width 0.508) (layer "B.Cu") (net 29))
 (segment (start 132.08 108.585) (end 116.3225 108.585) (width 0.508) (layer "B.Cu") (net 29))
 (segment (start 172.72 67.945) (end 132.08 108.585) (width 0.508) (layer "B.Cu") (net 29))
 (segment (start 188.2775 60.325) (end 180.34 60.325) (width 0.508) (layer "B.Cu") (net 32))
 (segment (start 132.08 100.965) (end 116.3225 100.965) (width 0.508) (layer "B.Cu") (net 32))
 (segment (start 172.72 60.325) (end 180.34 60.325) (width 0.25) (layer "B.Cu") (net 32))
 (segment (start 189.5475 59.055) (end 188.2775 60.325) (width 0.508) (layer "B.Cu") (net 32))
 (segment (start 191.77 59.055) (end 189.5475 59.055) (width 0.508) (layer "B.Cu") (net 32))
 (segment (start 172.72 60.325) (end 132.08 100.965) (width 0.508) (layer "B.Cu") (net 32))
 (segment (start 187.96 57.785) (end 189.23 56.515) (width 0.508) (layer "B.Cu") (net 33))
 (segment (start 116.3225 98.425) (end 132.08 98.425) (width 0.508) (layer "B.Cu") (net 33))
 (segment (start 172.72 57.785) (end 180.34 57.785) (width 0.25) (layer "B.Cu") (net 33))
 (segment (start 132.08 98.425) (end 172.72 57.785) (width 0.508) (layer "B.Cu") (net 33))
 (segment (start 189.23 56.515) (end 191.77 56.515) (width 0.508) (layer "B.Cu") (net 33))
 (segment (start 187.96 57.785) (end 180.34 57.785) (width 0.508) (layer "B.Cu") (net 33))
 (segment (start 132.08 95.885) (end 172.72 55.245) (width 0.508) (layer "B.Cu") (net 34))
 (segment (start 172.72 55.245) (end 180.34 55.245) (width 0.25) (layer "B.Cu") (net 34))
 (segment (start 188.2775 55.245) (end 180.34 55.245) (width 0.508) (layer "B.Cu") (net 34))
 (segment (start 191.77 53.975) (end 189.5475 53.975) (width 0.508) (layer "B.Cu") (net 34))
 (segment (start 189.5475 53.975) (end 188.2775 55.245) (width 0.508) (layer "B.Cu") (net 34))
 (segment (start 116.3225 95.885) (end 132.08 95.885) (width 0.508) (layer "B.Cu") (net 34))
 (segment (start 188.2775 52.705) (end 180.34 52.705) (width 0.508) (layer "B.Cu") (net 35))
 (segment (start 173.0375 52.705) (end 180.34 52.705) (width 0.25) (layer "B.Cu") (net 35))
 (segment (start 132.3975 93.345) (end 116.3225 93.345) (width 0.508) (layer "B.Cu") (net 35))
 (segment (start 173.0375 52.705) (end 132.3975 93.345) (width 0.508) (layer "B.Cu") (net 35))
 (segment (start 189.5475 51.435) (end 188.2775 52.705) (width 0.508) (layer "B.Cu") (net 35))
 (segment (start 191.77 51.435) (end 189.5475 51.435) (width 0.508) (layer "B.Cu") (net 35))
 (segment (start 172.72 50.165) (end 132.08 90.805) (width 0.508) (layer "B.Cu") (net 36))
 (segment (start 188.2775 50.165) (end 180.34 50.165) (width 0.508) (layer "B.Cu") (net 36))
 (segment (start 116.3225 90.805) (end 132.08 90.805) (width 0.508) (layer "B.Cu") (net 36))
 (segment (start 189.5475 48.895) (end 188.2775 50.165) (width 0.508) (layer "B.Cu") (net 36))
 (segment (start 191.77 48.895) (end 189.5475 48.895) (width 0.508) (layer "B.Cu") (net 36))
 (segment (start 172.72 50.165) (end 180.34 50.165) (width 0.25) (layer "B.Cu") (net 36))
 (segment (start 132.08 88.265) (end 172.72 47.625) (width 0.508) (layer "B.Cu") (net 37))
 (segment (start 188.2775 47.625) (end 180.34 47.625) (width 0.508) (layer "B.Cu") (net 37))
 (segment (start 188.2775 47.625) (end 189.5475 46.355) (width 0.508) (layer "B.Cu") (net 37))
 (segment (start 189.5475 46.355) (end 191.77 46.355) (width 0.508) (layer "B.Cu") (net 37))
 (segment (start 116.3225 88.265) (end 132.08 88.265) (width 0.508) (layer "B.Cu") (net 37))
 (segment (start 172.72 47.625) (end 180.34 47.625) (width 0.25) (layer "B.Cu") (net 37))
 (segment (start 172.72 45.085) (end 132.08 85.725) (width 0.508) (layer "B.Cu") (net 38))
 (segment (start 191.77 43.815) (end 189.5475 43.815) (width 0.508) (layer "B.Cu") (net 38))
 (segment (start 188.2775 45.085) (end 180.34 45.085) (width 0.508) (layer "B.Cu") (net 38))
 (segment (start 189.5475 43.815) (end 188.2775 45.085) (width 0.508) (layer "B.Cu") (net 38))
 (segment (start 116.3225 85.725) (end 132.08 85.725) (width 0.508) (layer "B.Cu") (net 38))
 (segment (start 172.72 45.085) (end 180.34 45.085) (width 0.25) (layer "B.Cu") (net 38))
 (segment (start 172.72 42.545) (end 132.08 83.185) (width 0.508) (layer "B.Cu") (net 39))
 (segment (start 132.08 83.185) (end 116.3225 83.185) (width 0.508) (layer "B.Cu") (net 39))
 (segment (start 188.2775 42.545) (end 180.34 42.545) (width 0.508) (layer "B.Cu") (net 39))
 (segment (start 191.77 41.275) (end 189.5475 41.275) (width 0.508) (layer "B.Cu") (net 39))
 (segment (start 172.72 42.545) (end 172.736 42.561) (width 0.508) (layer "B.Cu") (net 39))
 (segment (start 180.34 42.545) (end 180.324 42.561) (width 0.508) (layer "B.Cu") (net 39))
 (segment (start 172.736 42.561) (end 180.324 42.561) (width 0.25) (layer "B.Cu") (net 39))
 (segment (start 189.5475 41.275) (end 188.2775 42.545) (width 0.508) (layer "B.Cu") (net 39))
 (segment (start 132.08 80.645) (end 116.3225 80.645) (width 0.508) (layer "B.Cu") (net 40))
 (segment (start 188.2775 40.005) (end 180.34 40.005) (width 0.508) (layer "B.Cu") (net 40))
 (segment (start 191.77 38.735) (end 189.5475 38.735) (width 0.508) (layer "B.Cu") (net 40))
 (segment (start 189.5475 38.735) (end 188.2775 40.005) (width 0.508) (layer "B.Cu") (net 40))
 (segment (start 172.72 40.005) (end 132.08 80.645) (width 0.508) (layer "B.Cu") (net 40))
 (segment (start 172.72 40.005) (end 180.34 40.005) (width 0.25) (layer "B.Cu") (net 40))
 (segment (start 132.08 106.045) (end 116.3225 106.045) (width 0.508) (layer "B.Cu") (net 30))
 (segment (start 189.5475 64.135) (end 188.2775 65.405) (width 0.508) (layer "B.Cu") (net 30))
 (segment (start 172.72 65.405) (end 172.736 65.389) (width 0.508) (layer "B.Cu") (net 30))
 (segment (start 172.736 65.389) (end 180.324 65.389) (width 0.25) (layer "B.Cu") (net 30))
 (segment (start 172.72 65.405) (end 132.08 106.045) (width 0.508) (layer "B.Cu") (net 30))
 (segment (start 180.34 65.405) (end 180.324 65.389) (width 0.508) (layer "B.Cu") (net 30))
 (segment (start 188.2775 65.405) (end 180.34 65.405) (width 0.508) (layer "B.Cu") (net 30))
 (segment (start 191.77 64.135) (end 189.5475 64.135) (width 0.508) (layer "B.Cu") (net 30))
 (segment (start 191.77 61.595) (end 189.5475 61.595) (width 0.508) (layer "B.Cu") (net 31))
 (segment (start 132.08 103.505) (end 116.205 103.505) (width 0.508) (layer "B.Cu") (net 31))
 (segment (start 189.5475 61.595) (end 188.2775 62.865) (width 0.508) (layer "B.Cu") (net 31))
 (segment (start 188.2775 62.865) (end 180.34 62.865) (width 0.508) (layer "B.Cu") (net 31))
 (segment (start 172.72 62.865) (end 180.34 62.865) (width 0.25) (layer "B.Cu") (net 31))
 (segment (start 172.72 62.865) (end 132.08 103.505) (width 0.508) (layer "B.Cu") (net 31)))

